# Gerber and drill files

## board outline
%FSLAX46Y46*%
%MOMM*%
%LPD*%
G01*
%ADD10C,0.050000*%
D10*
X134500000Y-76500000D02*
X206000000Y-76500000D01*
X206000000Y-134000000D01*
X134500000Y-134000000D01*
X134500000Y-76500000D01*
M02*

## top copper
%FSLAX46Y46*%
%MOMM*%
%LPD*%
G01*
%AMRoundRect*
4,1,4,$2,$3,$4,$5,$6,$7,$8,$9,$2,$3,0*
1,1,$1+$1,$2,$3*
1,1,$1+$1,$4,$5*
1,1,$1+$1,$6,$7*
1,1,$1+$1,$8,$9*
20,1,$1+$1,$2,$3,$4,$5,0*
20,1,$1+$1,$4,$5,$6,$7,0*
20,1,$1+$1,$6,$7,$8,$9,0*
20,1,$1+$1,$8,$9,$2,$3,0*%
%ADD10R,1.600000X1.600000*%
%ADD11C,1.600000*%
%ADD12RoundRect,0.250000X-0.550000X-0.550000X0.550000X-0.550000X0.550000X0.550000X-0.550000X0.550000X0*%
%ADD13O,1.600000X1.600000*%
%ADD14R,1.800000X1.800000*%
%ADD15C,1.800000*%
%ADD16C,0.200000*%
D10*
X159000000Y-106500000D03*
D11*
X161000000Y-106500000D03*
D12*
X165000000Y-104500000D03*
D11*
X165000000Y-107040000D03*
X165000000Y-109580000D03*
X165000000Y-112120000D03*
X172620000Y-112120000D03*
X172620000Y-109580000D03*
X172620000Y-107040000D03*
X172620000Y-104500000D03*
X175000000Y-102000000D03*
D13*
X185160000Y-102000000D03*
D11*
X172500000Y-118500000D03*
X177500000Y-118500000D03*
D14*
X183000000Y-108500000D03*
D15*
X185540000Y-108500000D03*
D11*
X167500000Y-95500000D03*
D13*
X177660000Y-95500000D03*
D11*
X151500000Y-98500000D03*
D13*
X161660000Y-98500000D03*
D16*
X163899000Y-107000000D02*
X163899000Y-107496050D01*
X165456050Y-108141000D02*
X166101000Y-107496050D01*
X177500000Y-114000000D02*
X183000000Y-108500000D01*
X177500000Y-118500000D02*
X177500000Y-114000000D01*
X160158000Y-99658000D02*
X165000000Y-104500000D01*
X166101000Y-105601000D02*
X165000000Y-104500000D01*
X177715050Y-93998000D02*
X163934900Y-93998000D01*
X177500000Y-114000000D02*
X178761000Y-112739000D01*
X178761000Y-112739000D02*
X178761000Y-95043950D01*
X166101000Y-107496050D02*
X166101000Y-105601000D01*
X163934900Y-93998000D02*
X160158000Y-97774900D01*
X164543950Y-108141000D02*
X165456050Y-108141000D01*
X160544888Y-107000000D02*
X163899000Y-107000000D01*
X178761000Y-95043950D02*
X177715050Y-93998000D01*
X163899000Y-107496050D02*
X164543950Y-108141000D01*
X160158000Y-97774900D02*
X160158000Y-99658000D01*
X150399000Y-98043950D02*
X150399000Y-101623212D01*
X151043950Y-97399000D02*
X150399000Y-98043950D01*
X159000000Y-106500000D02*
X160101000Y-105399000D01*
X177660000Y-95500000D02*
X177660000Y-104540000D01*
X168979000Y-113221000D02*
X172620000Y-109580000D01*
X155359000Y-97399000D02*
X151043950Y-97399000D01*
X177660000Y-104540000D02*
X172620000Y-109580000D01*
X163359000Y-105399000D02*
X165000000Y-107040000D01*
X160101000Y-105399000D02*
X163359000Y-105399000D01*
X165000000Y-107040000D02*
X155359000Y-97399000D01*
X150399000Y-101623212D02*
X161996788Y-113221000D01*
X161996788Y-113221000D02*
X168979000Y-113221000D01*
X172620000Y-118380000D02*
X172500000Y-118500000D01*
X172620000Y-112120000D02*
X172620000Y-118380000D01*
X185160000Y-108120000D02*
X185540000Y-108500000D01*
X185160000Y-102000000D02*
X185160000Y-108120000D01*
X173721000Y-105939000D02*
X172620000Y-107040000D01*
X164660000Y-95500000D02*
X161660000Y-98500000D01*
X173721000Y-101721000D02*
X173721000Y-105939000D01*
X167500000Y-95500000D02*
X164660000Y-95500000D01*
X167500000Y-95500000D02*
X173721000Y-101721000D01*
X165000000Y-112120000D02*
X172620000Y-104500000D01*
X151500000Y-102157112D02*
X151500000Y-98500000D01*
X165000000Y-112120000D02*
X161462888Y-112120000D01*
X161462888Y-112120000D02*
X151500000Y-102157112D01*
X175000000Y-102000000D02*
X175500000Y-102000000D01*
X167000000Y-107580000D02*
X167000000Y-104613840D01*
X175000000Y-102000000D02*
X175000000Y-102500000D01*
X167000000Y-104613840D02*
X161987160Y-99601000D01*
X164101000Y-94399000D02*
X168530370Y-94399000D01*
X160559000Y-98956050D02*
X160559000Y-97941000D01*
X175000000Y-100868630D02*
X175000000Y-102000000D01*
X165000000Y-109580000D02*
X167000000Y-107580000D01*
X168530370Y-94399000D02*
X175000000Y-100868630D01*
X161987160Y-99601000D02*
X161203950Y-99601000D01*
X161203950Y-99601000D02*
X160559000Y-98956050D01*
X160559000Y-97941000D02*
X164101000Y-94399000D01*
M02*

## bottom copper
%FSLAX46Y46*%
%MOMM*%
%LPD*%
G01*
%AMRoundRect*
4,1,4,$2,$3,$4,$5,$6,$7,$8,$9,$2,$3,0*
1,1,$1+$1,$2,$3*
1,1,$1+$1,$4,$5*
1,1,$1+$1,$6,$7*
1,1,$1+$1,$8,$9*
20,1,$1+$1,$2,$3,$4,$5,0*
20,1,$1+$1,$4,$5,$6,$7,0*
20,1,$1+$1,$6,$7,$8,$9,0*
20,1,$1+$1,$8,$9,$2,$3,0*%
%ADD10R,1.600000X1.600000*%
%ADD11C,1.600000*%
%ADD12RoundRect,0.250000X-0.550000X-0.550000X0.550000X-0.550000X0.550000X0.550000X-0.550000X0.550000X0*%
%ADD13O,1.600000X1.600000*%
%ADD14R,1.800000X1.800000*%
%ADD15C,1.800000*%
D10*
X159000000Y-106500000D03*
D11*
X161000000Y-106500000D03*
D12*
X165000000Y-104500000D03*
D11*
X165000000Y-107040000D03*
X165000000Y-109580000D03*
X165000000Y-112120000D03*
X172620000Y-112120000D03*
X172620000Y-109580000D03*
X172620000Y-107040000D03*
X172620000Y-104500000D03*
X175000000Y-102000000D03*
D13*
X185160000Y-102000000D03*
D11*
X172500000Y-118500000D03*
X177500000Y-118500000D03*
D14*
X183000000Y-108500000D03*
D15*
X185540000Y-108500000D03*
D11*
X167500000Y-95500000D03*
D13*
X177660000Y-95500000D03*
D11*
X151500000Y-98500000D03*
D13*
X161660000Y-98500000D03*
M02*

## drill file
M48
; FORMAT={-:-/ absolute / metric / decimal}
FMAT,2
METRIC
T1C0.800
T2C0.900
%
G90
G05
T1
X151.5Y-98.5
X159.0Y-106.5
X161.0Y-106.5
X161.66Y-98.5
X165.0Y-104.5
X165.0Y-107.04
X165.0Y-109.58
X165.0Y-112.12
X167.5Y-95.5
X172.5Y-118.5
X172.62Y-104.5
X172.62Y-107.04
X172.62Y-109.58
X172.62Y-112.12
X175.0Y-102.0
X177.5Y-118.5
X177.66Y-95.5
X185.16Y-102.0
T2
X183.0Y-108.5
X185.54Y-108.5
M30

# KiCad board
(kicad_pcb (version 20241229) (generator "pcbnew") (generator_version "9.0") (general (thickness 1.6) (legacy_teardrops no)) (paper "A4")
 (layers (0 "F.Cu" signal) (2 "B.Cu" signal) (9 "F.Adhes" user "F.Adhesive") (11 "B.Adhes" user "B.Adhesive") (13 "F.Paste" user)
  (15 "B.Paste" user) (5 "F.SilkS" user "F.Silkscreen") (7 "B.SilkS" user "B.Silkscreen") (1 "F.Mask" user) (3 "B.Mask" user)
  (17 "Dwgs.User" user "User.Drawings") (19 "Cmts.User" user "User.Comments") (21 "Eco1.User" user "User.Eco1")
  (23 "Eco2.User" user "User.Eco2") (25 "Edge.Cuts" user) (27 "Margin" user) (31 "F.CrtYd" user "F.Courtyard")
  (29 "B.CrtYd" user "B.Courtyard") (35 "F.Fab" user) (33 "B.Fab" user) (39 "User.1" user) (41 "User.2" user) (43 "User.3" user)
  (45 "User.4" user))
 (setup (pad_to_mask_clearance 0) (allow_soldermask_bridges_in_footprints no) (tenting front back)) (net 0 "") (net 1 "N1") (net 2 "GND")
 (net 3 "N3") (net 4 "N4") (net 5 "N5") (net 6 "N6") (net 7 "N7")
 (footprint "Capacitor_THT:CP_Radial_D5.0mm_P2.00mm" (layer "F.Cu") (at 159 106.5)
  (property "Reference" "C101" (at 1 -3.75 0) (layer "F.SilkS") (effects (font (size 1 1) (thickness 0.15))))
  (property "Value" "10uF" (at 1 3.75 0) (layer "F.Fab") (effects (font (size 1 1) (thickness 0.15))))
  (pad "1" thru_hole rect (at 0 0) (size 1.6 1.6) (drill 0.8) (layers "*.Cu" "*.Mask") (remove_unused_layers no) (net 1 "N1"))
  (pad "2" thru_hole circle (at 2 0) (size 1.6 1.6) (drill 0.8) (layers "*.Cu" "*.Mask") (remove_unused_layers no) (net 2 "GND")))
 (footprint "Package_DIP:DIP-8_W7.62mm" (layer "F.Cu") (at 165 104.5)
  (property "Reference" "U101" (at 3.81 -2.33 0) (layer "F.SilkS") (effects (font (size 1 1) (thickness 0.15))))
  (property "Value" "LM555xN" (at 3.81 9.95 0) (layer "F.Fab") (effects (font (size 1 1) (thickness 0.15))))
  (pad "1" thru_hole roundrect (at 0 0) (size 1.6 1.6) (drill 0.8) (layers "*.Cu" "*.Mask") (remove_unused_layers no)
   (roundrect_rratio 0.15625) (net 2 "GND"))
  (pad "2" thru_hole circle (at 0 2.54) (size 1.6 1.6) (drill 0.8) (layers "*.Cu" "*.Mask") (remove_unused_layers no) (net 1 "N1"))
  (pad "3" thru_hole circle (at 0 5.08) (size 1.6 1.6) (drill 0.8) (layers "*.Cu" "*.Mask") (remove_unused_layers no) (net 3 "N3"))
  (pad "4" thru_hole circle (at 0 7.62) (size 1.6 1.6) (drill 0.8) (layers "*.Cu" "*.Mask") (remove_unused_layers no) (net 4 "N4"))
  (pad "5" thru_hole circle (at 7.62 7.62) (size 1.6 1.6) (drill 0.8) (layers "*.Cu" "*.Mask") (remove_unused_layers no) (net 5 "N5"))
  (pad "6" thru_hole circle (at 7.62 5.08) (size 1.6 1.6) (drill 0.8) (layers "*.Cu" "*.Mask") (remove_unused_layers no) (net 1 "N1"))
  (pad "7" thru_hole circle (at 7.62 2.54) (size 1.6 1.6) (drill 0.8) (layers "*.Cu" "*.Mask") (remove_unused_layers no) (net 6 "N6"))
  (pad "8" thru_hole circle (at 7.62 0) (size 1.6 1.6) (drill 0.8) (layers "*.Cu" "*.Mask") (remove_unused_layers no) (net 4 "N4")))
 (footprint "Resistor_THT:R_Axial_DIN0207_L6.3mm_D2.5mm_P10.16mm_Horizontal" (layer "F.Cu") (at 175 102)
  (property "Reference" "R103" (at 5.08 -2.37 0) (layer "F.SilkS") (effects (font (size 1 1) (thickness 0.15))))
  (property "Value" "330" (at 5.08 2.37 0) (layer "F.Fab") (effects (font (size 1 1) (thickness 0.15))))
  (pad "1" thru_hole circle (at 0 0) (size 1.6 1.6) (drill 0.8) (layers "*.Cu" "*.Mask") (remove_unused_layers no) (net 3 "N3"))
  (pad "2" thru_hole oval (at 10.16 0) (size 1.6 1.6) (drill 0.8) (layers "*.Cu" "*.Mask") (remove_unused_layers no) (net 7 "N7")))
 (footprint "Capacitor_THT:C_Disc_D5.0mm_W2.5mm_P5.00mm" (layer "F.Cu") (at 172.5 118.5)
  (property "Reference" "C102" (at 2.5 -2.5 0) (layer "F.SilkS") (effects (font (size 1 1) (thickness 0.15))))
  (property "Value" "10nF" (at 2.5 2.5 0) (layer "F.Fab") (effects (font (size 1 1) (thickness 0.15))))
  (pad "1" thru_hole circle (at 0 0) (size 1.6 1.6) (drill 0.8) (layers "*.Cu" "*.Mask") (remove_unused_layers no) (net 5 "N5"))
  (pad "2" thru_hole circle (at 5 0) (size 1.6 1.6) (drill 0.8) (layers "*.Cu" "*.Mask") (remove_unused_layers no) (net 2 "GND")))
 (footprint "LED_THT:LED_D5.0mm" (layer "F.Cu") (at 183 108.5)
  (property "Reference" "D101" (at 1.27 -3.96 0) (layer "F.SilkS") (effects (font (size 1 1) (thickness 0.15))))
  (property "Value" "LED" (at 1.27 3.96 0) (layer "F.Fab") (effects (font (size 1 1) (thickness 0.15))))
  (pad "1" thru_hole rect (at 0 0) (size 1.8 1.8) (drill 0.9) (layers "*.Cu" "*.Mask") (remove_unused_layers no) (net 2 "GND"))
  (pad "2" thru_hole circle (at 2.54 0) (size 1.8 1.8) (drill 0.9) (layers "*.Cu" "*.Mask") (remove_unused_layers no) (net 7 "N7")))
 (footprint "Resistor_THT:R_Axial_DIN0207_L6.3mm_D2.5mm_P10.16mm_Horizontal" (layer "F.Cu") (at 167.5 95.5)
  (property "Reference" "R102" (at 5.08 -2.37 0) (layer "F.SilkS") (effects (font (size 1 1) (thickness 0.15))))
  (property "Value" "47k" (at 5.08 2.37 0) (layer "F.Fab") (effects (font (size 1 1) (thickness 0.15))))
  (pad "1" thru_hole circle (at 0 0) (size 1.6 1.6) (drill 0.8) (layers "*.Cu" "*.Mask") (remove_unused_layers no) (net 6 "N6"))
  (pad "2" thru_hole oval (at 10.16 0) (size 1.6 1.6) (drill 0.8) (layers "*.Cu" "*.Mask") (remove_unused_layers no) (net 1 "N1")))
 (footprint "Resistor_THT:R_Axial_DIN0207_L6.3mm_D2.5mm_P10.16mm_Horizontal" (layer "F.Cu") (at 151.5 98.5)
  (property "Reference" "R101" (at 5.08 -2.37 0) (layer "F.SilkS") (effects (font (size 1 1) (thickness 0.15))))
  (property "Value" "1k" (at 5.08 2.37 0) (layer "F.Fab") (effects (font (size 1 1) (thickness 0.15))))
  (pad "1" thru_hole circle (at 0 0) (size 1.6 1.6) (drill 0.8) (layers "*.Cu" "*.Mask") (remove_unused_layers no) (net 4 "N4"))
  (pad "2" thru_hole oval (at 10.16 0) (size 1.6 1.6) (drill 0.8) (layers "*.Cu" "*.Mask") (remove_unused_layers no) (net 6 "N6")))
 (gr_rect (start 134.5 76.5) (end 206 134) (stroke (width 0.05) (type default)) (fill no) (layer "Edge.Cuts"))
 (segment (start 163.899 107) (end 163.899 107.49605) (width 0.2) (layer "F.Cu") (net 2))
 (segment (start 165.45605 108.141) (end 166.101 107.49605) (width 0.2) (layer "F.Cu") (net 2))
 (segment (start 177.5 114) (end 183 108.5) (width 0.2) (layer "F.Cu") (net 2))
 (segment (start 177.5 118.5) (end 177.5 114) (width 0.2) (layer "F.Cu") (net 2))
 (segment (start 160.158 99.658) (end 165 104.5) (width 0.2) (layer "F.Cu") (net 2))
 (segment (start 166.101 105.601) (end 165 104.5) (width 0.2) (layer "F.Cu") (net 2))
 (segment (start 177.71505 93.998) (end 163.9349 93.998) (width 0.2) (layer "F.Cu") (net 2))
 (segment (start 177.5 114) (end 178.761 112.739) (width 0.2) (layer "F.Cu") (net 2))
 (segment (start 178.761 112.739) (end 178.761 95.04395) (width 0.2) (layer "F.Cu") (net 2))
 (segment (start 166.101 107.49605) (end 166.101 105.601) (width 0.2) (layer "F.Cu") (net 2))
 (segment (start 163.9349 93.998) (end 160.158 97.7749) (width 0.2) (layer "F.Cu") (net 2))
 (segment (start 164.54395 108.141) (end 165.45605 108.141) (width 0.2) (layer "F.Cu") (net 2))
 (segment (start 160.544888 107) (end 163.899 107) (width 0.2) (layer "F.Cu") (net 2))
 (segment (start 178.761 95.04395) (end 177.71505 93.998) (width 0.2) (layer "F.Cu") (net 2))
 (segment (start 163.899 107.49605) (end 164.54395 108.141) (width 0.2) (layer "F.Cu") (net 2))
 (segment (start 160.158 97.7749) (end 160.158 99.658) (width 0.2) (layer "F.Cu") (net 2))
 (segment (start 150.399 98.04395) (end 150.399 101.623212) (width 0.2) (layer "F.Cu") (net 1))
 (segment (start 151.04395 97.399) (end 150.399 98.04395) (width 0.2) (layer "F.Cu") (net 1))
 (segment (start 159 106.5) (end 160.101 105.399) (width 0.2) (layer "F.Cu") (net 1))
 (segment (start 177.66 95.5) (end 177.66 104.54) (width 0.2) (layer "F.Cu") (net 1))
 (segment (start 168.979 113.221) (end 172.62 109.58) (width 0.2) (layer "F.Cu") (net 1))
 (segment (start 155.359 97.399) (end 151.04395 97.399) (width 0.2) (layer "F.Cu") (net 1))
 (segment (start 177.66 104.54) (end 172.62 109.58) (width 0.2) (layer "F.Cu") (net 1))
 (segment (start 163.359 105.399) (end 165 107.04) (width 0.2) (layer "F.Cu") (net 1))
 (segment (start 160.101 105.399) (end 163.359 105.399) (width 0.2) (layer "F.Cu") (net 1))
 (segment (start 165 107.04) (end 155.359 97.399) (width 0.2) (layer "F.Cu") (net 1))
 (segment (start 150.399 101.623212) (end 161.996788 113.221) (width 0.2) (layer "F.Cu") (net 1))
 (segment (start 161.996788 113.221) (end 168.979 113.221) (width 0.2) (layer "F.Cu") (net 1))
 (segment (start 172.62 118.38) (end 172.5 118.5) (width 0.2) (layer "F.Cu") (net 5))
 (segment (start 172.62 112.12) (end 172.62 118.38) (width 0.2) (layer "F.Cu") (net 5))
 (segment (start 185.16 108.12) (end 185.54 108.5) (width 0.2) (layer "F.Cu") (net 7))
 (segment (start 185.16 102) (end 185.16 108.12) (width 0.2) (layer "F.Cu") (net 7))
 (segment (start 173.721 105.939) (end 172.62 107.04) (width 0.2) (layer "F.Cu") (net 6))
 (segment (start 164.66 95.5) (end 161.66 98.5) (width 0.2) (layer "F.Cu") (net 6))
 (segment (start 173.721 101.721) (end 173.721 105.939) (width 0.2) (layer "F.Cu") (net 6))
 (segment (start 167.5 95.5) (end 164.66 95.5) (width 0.2) (layer "F.Cu") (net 6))
 (segment (start 167.5 95.5) (end 173.721 101.721) (width 0.2) (layer "F.Cu") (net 6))
 (segment (start 165 112.12) (end 172.62 104.5) (width 0.2) (layer "F.Cu") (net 4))
 (segment (start 151.5 102.157112) (end 151.5 98.5) (width 0.2) (layer "F.Cu") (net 4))
 (segment (start 165 112.12) (end 161.462888 112.12) (width 0.2) (layer "F.Cu") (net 4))
 (segment (start 161.462888 112.12) (end 151.5 102.157112) (width 0.2) (layer "F.Cu") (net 4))
 (segment (start 175 102) (end 175.5 102) (width 0.2) (layer "F.Cu") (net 3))
 (segment (start 167 107.58) (end 167 104.61384) (width 0.2) (layer "F.Cu") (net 3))
 (segment (start 175 102) (end 175 102.5) (width 0.2) (layer "F.Cu") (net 3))
 (segment (start 167 104.61384) (end 161.98716 99.601) (width 0.2) (layer "F.Cu") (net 3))
 (segment (start 164.101 94.399) (end 168.53037 94.399) (width 0.2) (layer "F.Cu") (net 3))
 (segment (start 160.559 98.95605) (end 160.559 97.941) (width 0.2) (layer "F.Cu") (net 3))
 (segment (start 175 100.86863) (end 175 102) (width 0.2) (layer "F.Cu") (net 3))
 (segment (start 165 109.58) (end 167 107.58) (width 0.2) (layer "F.Cu") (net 3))
 (segment (start 168.53037 94.399) (end 175 100.86863) (width 0.2) (layer "F.Cu") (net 3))
 (segment (start 161.98716 99.601) (end 161.20395 99.601) (width 0.2) (layer "F.Cu") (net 3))
 (segment (start 161.20395 99.601) (end 160.559 98.95605) (width 0.2) (layer "F.Cu") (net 3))
 (segment (start 160.559 97.941) (end 164.101 94.399) (width 0.2) (layer "F.Cu") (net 3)))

